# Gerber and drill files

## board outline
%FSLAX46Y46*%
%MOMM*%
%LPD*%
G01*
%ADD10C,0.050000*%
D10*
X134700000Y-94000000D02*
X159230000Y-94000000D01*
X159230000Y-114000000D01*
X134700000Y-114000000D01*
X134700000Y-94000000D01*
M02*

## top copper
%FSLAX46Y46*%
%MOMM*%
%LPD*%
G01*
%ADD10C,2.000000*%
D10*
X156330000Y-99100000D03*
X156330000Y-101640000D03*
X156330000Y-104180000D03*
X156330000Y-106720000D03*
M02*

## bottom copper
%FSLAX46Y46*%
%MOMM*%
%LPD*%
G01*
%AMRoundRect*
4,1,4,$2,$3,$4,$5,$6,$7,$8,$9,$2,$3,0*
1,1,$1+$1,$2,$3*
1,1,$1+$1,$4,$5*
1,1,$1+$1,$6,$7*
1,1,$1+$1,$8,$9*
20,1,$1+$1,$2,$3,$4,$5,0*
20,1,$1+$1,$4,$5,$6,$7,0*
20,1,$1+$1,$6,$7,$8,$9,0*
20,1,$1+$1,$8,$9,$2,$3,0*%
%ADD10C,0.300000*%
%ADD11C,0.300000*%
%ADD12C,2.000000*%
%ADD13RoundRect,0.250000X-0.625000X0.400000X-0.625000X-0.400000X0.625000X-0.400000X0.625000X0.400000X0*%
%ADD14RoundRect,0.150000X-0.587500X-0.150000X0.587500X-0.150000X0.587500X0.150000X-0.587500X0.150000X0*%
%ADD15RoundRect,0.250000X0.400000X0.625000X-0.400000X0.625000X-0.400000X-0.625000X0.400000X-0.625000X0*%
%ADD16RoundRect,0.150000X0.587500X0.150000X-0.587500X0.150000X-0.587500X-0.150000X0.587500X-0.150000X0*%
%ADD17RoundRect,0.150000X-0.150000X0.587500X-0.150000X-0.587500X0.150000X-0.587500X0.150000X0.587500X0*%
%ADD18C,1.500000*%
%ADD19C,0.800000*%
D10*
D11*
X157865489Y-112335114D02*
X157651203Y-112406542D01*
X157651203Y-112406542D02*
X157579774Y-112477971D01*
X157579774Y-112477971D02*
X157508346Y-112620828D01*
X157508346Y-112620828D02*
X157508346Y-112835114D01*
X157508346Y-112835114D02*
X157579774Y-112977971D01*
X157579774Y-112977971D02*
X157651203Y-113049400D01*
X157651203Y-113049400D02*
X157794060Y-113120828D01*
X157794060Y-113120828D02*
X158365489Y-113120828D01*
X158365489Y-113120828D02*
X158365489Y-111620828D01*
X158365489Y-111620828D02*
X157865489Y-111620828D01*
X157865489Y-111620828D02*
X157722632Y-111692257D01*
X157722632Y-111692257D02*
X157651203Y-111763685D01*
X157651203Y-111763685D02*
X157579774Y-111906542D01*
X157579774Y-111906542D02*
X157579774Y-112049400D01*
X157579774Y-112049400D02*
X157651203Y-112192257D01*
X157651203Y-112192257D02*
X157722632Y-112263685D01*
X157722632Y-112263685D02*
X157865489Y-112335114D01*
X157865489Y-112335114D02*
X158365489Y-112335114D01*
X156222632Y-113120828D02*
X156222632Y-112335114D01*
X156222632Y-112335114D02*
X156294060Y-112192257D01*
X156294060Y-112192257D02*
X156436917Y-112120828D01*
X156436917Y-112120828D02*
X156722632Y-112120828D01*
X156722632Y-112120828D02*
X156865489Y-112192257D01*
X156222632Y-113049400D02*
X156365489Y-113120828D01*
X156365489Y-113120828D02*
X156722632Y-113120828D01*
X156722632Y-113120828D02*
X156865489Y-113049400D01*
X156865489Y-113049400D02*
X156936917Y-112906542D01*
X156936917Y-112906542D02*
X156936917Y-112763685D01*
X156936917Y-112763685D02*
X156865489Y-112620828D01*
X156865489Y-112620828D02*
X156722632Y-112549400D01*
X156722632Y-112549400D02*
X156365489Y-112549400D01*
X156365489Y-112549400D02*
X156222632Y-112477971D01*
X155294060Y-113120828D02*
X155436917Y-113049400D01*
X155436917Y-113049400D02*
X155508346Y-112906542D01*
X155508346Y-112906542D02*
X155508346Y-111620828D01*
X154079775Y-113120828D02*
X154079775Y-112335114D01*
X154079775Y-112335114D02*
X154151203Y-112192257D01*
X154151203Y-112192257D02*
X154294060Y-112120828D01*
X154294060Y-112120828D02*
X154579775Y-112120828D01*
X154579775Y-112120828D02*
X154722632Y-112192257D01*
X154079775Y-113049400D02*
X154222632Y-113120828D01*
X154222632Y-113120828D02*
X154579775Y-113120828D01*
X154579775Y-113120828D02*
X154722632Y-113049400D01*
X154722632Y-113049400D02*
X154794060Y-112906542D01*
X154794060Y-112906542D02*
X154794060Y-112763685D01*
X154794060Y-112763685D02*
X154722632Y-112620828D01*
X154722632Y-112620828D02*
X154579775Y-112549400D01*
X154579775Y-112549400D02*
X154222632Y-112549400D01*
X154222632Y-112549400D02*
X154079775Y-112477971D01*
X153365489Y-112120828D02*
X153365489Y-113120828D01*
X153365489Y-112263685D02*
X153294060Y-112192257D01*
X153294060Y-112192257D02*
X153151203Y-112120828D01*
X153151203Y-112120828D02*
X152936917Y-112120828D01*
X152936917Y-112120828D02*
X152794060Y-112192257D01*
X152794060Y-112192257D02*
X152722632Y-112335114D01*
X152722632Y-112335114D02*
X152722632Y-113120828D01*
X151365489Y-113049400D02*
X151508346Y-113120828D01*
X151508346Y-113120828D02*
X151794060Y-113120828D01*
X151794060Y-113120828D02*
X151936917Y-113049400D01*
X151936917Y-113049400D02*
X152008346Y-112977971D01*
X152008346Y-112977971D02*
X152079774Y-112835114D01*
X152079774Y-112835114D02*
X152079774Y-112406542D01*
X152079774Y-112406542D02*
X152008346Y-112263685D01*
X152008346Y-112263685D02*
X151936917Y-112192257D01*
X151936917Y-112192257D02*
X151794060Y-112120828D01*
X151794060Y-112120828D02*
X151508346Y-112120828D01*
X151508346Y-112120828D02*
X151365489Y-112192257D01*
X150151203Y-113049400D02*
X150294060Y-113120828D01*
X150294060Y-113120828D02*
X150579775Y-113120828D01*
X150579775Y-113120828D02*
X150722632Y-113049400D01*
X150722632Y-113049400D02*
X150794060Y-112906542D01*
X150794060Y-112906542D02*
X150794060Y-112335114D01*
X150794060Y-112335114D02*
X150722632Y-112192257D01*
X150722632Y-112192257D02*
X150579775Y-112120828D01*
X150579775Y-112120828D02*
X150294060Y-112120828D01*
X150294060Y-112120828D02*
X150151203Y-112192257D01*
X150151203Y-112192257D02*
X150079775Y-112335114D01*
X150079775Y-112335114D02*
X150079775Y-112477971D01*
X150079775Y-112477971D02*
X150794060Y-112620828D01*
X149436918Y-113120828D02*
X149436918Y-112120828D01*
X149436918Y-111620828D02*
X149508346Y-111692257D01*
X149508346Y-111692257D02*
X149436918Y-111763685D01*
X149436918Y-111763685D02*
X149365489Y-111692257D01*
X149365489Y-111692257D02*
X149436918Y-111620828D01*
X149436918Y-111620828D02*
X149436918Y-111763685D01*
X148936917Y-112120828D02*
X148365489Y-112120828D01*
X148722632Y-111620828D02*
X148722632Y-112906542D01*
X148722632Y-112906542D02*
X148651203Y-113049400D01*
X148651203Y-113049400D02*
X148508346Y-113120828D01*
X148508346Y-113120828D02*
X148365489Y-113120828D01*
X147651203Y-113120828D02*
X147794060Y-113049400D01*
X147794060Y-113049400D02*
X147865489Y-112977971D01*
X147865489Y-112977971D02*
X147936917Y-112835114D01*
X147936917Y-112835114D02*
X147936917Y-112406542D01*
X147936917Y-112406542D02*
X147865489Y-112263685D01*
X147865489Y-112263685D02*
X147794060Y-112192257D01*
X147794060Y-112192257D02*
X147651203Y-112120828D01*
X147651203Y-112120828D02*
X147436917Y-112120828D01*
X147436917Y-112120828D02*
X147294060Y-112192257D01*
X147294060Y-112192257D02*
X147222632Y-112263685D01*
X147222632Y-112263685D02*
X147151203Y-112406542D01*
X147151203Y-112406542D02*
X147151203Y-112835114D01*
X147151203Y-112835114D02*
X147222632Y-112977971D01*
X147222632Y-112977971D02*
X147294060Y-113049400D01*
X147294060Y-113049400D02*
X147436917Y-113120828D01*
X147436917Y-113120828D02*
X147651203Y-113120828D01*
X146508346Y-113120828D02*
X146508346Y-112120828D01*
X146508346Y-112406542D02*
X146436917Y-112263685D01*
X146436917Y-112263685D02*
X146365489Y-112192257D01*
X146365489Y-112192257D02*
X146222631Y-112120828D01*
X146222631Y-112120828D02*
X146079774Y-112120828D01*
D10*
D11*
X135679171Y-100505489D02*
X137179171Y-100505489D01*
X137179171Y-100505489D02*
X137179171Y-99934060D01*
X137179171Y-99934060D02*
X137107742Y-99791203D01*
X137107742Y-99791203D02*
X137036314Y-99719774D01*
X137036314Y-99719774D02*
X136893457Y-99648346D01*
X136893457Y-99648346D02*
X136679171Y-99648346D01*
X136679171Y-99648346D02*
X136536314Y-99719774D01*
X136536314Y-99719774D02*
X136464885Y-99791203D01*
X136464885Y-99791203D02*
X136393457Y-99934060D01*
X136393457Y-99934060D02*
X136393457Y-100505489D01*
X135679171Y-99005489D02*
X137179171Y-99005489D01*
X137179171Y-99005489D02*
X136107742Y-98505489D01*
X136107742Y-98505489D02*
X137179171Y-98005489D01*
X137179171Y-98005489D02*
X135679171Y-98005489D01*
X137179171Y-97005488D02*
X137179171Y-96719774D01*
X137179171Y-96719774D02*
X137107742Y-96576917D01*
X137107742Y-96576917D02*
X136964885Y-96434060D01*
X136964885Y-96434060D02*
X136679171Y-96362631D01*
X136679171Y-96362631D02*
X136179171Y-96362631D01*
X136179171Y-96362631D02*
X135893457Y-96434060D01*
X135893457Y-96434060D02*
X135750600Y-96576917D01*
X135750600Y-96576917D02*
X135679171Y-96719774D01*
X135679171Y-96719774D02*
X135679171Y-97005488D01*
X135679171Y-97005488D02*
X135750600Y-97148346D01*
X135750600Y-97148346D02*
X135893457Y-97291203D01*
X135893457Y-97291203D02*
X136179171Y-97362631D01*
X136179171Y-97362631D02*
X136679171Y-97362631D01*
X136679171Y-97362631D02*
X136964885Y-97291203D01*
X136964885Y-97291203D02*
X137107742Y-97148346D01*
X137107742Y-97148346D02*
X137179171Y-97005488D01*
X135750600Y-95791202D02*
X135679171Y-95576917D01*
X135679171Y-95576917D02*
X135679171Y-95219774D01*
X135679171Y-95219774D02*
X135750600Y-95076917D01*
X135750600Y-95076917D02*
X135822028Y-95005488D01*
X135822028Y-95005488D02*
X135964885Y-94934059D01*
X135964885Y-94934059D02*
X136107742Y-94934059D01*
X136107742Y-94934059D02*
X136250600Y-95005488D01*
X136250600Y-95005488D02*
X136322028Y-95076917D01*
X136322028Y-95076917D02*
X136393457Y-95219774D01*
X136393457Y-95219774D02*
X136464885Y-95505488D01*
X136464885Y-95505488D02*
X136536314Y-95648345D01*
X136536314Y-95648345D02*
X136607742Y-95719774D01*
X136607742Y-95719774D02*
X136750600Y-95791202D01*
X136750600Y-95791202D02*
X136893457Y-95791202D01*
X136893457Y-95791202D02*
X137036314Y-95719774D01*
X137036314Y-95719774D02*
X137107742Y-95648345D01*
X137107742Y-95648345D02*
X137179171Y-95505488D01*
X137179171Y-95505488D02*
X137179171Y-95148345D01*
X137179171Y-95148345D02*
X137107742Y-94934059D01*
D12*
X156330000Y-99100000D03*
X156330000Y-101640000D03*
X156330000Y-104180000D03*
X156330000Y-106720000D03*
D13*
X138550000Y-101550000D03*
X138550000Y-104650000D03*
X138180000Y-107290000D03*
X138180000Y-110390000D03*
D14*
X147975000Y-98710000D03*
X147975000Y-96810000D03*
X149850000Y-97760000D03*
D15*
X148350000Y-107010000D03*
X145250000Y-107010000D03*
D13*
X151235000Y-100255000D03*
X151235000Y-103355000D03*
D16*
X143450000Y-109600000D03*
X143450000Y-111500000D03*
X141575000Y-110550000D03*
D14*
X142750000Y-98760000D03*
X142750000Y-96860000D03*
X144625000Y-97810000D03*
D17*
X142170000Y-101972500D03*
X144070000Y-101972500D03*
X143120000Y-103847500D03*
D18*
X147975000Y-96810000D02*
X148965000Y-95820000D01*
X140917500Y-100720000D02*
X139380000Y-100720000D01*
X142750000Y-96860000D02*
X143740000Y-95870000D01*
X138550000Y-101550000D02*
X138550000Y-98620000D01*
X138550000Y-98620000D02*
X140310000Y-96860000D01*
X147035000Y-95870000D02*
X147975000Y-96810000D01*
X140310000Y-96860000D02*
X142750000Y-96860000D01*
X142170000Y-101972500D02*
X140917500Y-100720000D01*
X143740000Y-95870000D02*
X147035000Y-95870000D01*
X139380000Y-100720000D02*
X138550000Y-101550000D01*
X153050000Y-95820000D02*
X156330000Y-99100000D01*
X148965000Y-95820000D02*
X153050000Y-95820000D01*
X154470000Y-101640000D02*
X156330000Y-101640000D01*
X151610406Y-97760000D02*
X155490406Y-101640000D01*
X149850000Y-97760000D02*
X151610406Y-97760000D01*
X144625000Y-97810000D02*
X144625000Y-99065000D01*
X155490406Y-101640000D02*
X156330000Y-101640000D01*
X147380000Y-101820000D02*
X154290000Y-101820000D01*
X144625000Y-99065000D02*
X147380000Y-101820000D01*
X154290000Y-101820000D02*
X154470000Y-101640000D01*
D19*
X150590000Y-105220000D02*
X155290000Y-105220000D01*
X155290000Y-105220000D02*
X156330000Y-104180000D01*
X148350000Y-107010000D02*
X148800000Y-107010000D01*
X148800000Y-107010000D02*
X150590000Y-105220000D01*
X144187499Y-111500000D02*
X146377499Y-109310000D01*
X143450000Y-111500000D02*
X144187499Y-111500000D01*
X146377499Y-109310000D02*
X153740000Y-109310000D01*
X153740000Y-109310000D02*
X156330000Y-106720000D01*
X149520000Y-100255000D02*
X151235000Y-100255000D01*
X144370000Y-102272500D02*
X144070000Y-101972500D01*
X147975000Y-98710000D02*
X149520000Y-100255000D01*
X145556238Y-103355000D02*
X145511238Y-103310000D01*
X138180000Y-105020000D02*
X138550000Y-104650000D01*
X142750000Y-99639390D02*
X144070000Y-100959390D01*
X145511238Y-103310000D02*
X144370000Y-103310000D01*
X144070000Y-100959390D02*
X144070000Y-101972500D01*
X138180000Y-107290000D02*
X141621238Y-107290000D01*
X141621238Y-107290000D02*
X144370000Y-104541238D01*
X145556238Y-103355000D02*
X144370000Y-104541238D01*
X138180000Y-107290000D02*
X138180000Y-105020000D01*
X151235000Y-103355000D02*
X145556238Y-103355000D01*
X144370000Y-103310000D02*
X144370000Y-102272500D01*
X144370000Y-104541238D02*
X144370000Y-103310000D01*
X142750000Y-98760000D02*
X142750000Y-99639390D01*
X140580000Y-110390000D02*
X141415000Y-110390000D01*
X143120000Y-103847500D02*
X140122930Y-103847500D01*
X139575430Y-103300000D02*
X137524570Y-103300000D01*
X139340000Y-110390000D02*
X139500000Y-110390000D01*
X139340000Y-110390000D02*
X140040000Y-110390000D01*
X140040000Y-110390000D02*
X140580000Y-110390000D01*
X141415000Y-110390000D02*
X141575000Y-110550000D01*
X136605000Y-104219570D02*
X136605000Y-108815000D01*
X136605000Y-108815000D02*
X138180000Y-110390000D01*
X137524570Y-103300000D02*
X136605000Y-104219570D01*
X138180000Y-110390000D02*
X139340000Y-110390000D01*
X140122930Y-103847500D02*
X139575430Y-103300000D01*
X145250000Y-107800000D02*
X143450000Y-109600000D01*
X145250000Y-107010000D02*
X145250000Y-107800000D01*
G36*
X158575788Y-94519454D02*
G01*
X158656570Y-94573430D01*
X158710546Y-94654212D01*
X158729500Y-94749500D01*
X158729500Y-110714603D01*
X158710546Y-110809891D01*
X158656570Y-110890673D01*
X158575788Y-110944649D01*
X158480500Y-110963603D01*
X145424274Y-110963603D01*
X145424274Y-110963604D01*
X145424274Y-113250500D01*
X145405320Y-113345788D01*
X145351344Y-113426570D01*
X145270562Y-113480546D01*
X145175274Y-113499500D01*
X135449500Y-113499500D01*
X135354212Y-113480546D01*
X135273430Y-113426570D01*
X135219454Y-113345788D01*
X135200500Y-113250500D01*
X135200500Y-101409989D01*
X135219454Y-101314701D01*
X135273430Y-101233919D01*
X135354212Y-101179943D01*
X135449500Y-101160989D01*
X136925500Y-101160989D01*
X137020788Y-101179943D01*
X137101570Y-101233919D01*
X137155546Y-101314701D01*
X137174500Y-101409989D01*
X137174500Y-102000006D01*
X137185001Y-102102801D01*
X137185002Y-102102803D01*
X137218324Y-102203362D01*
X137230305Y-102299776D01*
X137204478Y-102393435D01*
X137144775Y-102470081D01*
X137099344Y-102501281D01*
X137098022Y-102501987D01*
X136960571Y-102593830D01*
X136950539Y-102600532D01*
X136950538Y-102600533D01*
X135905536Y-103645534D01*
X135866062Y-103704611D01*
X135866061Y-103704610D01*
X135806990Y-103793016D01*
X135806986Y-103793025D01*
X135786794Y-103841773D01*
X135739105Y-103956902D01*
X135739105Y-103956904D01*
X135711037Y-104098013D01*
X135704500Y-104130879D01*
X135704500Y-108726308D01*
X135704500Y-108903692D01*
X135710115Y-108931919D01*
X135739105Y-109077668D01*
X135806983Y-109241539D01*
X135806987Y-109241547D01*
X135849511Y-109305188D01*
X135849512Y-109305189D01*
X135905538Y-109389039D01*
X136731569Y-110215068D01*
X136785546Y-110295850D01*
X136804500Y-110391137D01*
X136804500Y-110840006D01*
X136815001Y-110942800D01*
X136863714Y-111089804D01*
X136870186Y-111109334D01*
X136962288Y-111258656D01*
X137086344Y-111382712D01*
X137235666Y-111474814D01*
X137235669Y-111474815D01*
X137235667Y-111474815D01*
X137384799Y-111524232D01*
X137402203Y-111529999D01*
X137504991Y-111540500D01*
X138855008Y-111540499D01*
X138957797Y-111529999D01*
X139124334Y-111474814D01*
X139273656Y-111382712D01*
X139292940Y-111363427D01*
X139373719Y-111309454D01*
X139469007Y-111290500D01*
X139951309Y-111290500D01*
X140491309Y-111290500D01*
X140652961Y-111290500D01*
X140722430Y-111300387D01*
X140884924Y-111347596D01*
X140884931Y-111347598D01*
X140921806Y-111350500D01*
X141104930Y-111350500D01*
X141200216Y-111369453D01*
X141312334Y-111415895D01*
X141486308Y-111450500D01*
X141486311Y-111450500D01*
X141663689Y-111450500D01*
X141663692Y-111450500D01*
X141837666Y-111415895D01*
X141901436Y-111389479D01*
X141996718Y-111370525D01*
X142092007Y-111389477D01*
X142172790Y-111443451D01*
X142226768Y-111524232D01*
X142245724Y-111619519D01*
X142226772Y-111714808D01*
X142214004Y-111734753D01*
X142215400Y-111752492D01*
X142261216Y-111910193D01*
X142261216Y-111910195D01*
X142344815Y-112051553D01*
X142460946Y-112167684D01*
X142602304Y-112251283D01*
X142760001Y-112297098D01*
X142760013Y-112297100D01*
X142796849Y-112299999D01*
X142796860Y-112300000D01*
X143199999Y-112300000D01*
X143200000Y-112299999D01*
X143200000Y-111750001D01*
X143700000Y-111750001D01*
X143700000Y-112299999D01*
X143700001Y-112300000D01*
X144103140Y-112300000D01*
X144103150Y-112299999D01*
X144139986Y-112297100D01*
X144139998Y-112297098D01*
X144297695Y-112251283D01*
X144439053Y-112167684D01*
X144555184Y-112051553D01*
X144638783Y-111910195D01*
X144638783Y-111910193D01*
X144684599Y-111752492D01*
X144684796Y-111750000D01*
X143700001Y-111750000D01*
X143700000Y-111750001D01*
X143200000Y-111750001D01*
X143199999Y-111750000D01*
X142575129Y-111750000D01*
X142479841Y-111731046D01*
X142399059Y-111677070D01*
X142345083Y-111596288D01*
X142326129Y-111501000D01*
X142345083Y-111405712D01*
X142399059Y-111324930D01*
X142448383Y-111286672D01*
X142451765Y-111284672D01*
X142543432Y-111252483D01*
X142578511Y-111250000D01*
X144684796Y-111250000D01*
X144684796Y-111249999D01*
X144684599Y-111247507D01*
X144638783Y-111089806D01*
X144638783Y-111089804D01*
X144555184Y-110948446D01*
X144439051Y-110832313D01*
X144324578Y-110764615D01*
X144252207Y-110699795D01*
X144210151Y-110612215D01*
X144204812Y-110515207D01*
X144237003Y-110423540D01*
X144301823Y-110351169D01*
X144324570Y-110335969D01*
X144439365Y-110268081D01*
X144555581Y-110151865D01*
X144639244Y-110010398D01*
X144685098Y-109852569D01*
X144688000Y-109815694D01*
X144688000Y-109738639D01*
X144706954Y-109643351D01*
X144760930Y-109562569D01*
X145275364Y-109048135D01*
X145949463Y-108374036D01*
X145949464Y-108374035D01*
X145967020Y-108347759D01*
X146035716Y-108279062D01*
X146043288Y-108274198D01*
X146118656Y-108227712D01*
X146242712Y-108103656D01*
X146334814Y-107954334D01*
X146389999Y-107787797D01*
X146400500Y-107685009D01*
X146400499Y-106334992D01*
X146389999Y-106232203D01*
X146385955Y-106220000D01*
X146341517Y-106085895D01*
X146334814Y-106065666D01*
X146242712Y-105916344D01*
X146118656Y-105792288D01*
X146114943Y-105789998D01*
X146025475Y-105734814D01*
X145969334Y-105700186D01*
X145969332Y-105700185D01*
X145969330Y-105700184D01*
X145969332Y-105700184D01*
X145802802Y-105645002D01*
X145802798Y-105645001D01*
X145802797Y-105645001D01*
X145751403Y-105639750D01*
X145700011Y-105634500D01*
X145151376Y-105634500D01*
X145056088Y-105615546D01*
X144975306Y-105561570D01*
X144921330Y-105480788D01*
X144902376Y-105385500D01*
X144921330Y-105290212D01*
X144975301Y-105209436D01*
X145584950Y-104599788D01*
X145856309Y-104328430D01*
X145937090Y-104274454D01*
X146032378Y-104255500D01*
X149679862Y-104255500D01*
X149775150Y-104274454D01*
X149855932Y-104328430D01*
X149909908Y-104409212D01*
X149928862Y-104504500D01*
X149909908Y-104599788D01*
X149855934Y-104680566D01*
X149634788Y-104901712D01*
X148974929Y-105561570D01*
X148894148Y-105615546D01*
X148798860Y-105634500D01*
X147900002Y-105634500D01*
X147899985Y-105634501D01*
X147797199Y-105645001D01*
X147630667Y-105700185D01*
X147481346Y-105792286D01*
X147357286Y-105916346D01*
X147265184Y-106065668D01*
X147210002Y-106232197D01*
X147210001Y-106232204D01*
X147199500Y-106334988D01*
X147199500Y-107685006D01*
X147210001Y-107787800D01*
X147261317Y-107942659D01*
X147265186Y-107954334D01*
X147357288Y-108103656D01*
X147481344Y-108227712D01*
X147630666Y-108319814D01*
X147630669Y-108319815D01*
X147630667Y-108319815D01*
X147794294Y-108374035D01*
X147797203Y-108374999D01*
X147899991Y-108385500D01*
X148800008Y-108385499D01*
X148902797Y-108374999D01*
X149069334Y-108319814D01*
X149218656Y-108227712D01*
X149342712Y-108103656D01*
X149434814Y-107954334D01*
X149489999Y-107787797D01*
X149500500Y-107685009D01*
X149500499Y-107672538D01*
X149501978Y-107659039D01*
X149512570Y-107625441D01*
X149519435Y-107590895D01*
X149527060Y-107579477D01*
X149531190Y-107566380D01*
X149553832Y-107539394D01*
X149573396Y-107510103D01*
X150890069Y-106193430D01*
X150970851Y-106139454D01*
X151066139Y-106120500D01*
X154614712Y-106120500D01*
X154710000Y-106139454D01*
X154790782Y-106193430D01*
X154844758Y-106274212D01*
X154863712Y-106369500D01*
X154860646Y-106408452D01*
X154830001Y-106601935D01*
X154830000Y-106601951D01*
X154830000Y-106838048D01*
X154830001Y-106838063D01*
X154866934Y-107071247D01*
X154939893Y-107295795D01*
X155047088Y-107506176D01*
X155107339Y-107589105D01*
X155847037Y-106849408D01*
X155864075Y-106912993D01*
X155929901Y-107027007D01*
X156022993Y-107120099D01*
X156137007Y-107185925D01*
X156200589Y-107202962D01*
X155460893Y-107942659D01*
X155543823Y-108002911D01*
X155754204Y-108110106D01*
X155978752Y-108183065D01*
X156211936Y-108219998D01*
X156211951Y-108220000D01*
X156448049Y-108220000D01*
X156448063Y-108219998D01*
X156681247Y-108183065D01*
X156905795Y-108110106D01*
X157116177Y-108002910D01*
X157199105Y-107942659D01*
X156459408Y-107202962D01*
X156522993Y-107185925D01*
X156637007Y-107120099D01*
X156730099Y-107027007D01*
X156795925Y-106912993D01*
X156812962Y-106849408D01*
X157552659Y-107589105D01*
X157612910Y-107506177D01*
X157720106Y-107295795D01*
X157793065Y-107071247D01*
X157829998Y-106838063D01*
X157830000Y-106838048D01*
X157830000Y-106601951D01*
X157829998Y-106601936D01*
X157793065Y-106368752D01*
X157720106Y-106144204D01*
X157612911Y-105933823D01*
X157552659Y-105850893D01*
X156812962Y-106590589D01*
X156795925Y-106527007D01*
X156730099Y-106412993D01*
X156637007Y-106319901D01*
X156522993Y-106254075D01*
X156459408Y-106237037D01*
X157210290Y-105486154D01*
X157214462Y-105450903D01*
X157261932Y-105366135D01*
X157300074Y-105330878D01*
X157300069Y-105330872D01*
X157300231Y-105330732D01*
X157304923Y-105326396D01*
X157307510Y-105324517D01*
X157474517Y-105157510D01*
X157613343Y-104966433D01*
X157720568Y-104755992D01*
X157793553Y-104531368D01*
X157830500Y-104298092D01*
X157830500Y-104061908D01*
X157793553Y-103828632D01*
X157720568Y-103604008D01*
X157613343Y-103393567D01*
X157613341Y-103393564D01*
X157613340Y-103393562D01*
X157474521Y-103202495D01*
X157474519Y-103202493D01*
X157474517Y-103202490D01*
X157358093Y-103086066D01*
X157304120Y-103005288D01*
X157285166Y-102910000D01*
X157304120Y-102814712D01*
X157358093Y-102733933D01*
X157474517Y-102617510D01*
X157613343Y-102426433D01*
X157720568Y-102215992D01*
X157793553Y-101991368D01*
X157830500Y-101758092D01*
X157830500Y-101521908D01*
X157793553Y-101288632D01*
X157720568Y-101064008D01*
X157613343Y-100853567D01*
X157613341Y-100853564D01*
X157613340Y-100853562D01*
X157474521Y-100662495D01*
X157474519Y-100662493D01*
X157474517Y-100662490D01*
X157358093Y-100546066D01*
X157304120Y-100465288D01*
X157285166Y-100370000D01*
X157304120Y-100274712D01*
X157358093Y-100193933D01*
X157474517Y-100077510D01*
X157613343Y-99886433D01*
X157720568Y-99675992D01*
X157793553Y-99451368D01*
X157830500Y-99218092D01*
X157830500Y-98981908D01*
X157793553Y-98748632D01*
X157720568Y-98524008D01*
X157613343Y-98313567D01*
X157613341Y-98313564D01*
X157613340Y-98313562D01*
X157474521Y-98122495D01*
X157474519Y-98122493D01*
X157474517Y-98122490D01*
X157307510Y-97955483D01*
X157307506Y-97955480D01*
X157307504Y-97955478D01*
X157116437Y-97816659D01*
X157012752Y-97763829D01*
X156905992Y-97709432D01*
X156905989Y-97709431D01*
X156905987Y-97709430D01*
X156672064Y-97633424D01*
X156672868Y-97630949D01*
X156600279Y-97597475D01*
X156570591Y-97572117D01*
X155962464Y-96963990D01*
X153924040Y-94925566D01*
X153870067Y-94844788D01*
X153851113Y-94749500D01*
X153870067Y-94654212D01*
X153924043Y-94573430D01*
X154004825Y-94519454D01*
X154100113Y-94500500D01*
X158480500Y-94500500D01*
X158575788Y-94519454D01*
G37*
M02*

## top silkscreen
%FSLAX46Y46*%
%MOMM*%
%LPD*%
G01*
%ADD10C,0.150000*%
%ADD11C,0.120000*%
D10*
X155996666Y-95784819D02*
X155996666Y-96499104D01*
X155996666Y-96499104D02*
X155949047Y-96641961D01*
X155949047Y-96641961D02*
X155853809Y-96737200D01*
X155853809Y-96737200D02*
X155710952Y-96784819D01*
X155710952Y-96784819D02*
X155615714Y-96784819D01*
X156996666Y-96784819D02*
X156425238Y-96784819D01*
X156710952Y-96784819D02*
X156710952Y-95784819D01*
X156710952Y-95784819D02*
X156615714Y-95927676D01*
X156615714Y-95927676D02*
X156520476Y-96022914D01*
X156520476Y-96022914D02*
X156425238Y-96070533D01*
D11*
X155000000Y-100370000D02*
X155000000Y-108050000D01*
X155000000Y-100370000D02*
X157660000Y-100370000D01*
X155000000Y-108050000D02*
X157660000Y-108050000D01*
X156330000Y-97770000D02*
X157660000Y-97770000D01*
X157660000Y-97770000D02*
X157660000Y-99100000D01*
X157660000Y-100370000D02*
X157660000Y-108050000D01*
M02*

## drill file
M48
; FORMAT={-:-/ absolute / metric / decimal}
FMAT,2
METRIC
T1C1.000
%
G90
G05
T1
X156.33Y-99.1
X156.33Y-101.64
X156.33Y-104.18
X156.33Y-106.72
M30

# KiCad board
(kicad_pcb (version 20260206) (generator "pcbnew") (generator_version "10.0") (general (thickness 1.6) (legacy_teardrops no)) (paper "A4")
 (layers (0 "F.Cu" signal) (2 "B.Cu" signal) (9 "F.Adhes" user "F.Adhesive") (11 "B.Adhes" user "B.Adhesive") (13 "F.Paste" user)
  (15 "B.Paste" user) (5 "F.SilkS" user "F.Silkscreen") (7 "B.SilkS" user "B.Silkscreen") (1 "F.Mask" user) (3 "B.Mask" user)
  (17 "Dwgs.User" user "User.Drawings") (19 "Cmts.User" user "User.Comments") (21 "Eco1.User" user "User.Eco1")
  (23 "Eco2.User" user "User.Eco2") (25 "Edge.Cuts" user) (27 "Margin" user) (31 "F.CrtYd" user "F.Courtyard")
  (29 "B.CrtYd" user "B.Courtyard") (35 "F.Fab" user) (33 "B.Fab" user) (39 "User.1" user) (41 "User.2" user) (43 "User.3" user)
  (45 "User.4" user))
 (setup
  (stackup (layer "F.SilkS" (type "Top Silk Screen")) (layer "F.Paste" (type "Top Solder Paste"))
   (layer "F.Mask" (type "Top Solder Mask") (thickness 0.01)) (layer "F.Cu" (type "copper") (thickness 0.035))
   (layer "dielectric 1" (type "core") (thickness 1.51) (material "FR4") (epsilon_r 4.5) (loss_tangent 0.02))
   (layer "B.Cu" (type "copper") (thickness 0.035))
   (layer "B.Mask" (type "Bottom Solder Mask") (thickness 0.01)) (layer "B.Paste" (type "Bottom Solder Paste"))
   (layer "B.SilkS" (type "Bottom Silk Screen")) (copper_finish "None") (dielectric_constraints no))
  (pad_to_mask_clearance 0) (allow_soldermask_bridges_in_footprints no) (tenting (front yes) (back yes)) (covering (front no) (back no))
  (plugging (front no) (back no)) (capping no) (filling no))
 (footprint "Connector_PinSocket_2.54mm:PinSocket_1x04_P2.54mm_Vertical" (layer "F.Cu") (at 156.33 99.1)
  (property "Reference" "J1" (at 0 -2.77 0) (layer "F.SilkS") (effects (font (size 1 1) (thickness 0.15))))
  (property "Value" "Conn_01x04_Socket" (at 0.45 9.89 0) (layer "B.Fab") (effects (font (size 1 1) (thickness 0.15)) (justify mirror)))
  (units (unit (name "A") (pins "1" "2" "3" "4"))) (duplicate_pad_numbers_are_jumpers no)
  (fp_line (start -1.33 1.27) (end -1.33 8.95) (stroke (width 0.12) (type solid)) (layer "F.SilkS"))
  (fp_line (start -1.33 1.27) (end 1.33 1.27) (stroke (width 0.12) (type solid)) (layer "F.SilkS"))
  (fp_line (start -1.33 8.95) (end 1.33 8.95) (stroke (width 0.12) (type solid)) (layer "F.SilkS"))
  (fp_line (start 0 -1.33) (end 1.33 -1.33) (stroke (width 0.12) (type solid)) (layer "F.SilkS"))
  (fp_line (start 1.33 -1.33) (end 1.33 0) (stroke (width 0.12) (type solid)) (layer "F.SilkS"))
  (fp_line (start 1.33 1.27) (end 1.33 8.95) (stroke (width 0.12) (type solid)) (layer "F.SilkS"))
  (pad "1" thru_hole circle (at 0 0) (size 2 2) (drill 1) (layers "*.Cu" "*.Mask") (remove_unused_layers no) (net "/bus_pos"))
  (pad "2" thru_hole circle (at 0 2.54) (size 2 2) (drill 1) (layers "*.Cu" "*.Mask") (remove_unused_layers no) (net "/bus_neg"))
  (pad "3" thru_hole circle (at 0 5.08) (size 2 2) (drill 1) (layers "*.Cu" "*.Mask") (remove_unused_layers no) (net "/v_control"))
  (pad "4" thru_hole circle (at 0 7.62) (size 2 2) (drill 1) (layers "*.Cu" "*.Mask") (remove_unused_layers no) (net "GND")))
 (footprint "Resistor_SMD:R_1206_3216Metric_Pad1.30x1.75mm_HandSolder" (layer "B.Cu") (at 138.55 103.1 -90)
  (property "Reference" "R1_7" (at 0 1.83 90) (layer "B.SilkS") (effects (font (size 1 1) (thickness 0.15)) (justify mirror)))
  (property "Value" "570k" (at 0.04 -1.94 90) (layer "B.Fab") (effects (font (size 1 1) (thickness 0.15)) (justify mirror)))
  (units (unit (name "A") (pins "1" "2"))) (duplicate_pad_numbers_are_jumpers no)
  (pad "1" smd roundrect (at -1.55 0 270) (size 1.3 1.75) (layers "B.Cu" "B.Mask" "B.Paste") (roundrect_rratio 0.192308) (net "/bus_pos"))
  (pad "2" smd roundrect (at 1.55 0 270) (size 1.3 1.75) (layers "B.Cu" "B.Mask" "B.Paste") (roundrect_rratio 0.192308) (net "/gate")))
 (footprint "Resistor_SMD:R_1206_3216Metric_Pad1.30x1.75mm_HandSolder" (layer "B.Cu") (at 138.18 108.84 -90)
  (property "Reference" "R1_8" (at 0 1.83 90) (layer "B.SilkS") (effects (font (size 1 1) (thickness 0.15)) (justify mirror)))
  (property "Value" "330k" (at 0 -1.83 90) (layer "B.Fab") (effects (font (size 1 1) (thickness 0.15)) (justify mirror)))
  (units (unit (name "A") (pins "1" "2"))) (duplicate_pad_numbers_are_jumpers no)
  (pad "1" smd roundrect (at -1.55 0 270) (size 1.3 1.75) (layers "B.Cu" "B.Mask" "B.Paste") (roundrect_rratio 0.192308) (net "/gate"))
  (pad "2" smd roundrect (at 1.55 0 270) (size 1.3 1.75) (layers "B.Cu" "B.Mask" "B.Paste") (roundrect_rratio 0.192308) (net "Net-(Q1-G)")))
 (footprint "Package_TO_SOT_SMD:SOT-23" (layer "B.Cu") (at 148.9125 97.76)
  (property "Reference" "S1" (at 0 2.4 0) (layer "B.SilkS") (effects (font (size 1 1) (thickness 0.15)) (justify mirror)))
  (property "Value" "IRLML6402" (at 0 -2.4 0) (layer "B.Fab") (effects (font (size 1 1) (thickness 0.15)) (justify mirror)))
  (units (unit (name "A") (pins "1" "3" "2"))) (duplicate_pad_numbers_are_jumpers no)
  (pad "1" smd roundrect (at -0.9375 0.95) (size 1.475 0.6) (layers "B.Cu" "B.Mask" "B.Paste") (roundrect_rratio 0.25) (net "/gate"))
  (pad "2" smd roundrect (at -0.9375 -0.95) (size 1.475 0.6) (layers "B.Cu" "B.Mask" "B.Paste") (roundrect_rratio 0.25) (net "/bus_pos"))
  (pad "3" smd roundrect (at 0.9375 0) (size 1.475 0.6) (layers "B.Cu" "B.Mask" "B.Paste") (roundrect_rratio 0.25) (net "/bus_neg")))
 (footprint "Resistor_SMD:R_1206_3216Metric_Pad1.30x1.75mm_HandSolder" (layer "B.Cu") (at 146.8 107.01 180)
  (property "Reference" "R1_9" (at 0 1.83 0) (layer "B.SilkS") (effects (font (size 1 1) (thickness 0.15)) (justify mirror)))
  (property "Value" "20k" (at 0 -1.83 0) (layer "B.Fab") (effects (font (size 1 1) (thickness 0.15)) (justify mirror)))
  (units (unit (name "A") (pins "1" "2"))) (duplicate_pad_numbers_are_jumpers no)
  (pad "1" smd roundrect (at -1.55 0 180) (size 1.3 1.75) (layers "B.Cu" "B.Mask" "B.Paste") (roundrect_rratio 0.192308) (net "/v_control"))
  (pad "2" smd roundrect (at 1.55 0 180) (size 1.3 1.75) (layers "B.Cu" "B.Mask" "B.Paste") (roundrect_rratio 0.192308) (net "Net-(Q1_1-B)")))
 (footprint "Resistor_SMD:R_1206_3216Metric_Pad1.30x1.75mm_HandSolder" (layer "B.Cu") (at 151.235 101.805 -90)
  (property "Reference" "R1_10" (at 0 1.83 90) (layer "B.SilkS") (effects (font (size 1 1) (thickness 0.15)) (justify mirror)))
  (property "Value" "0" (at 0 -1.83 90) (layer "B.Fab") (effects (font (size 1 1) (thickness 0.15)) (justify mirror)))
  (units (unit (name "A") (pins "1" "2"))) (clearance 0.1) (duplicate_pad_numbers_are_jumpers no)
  (pad "1" smd roundrect (at -1.55 0 270) (size 1.3 1.75) (layers "B.Cu" "B.Mask" "B.Paste") (roundrect_rratio 0.192308) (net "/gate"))
  (pad "2" smd roundrect (at 1.55 0 270) (size 1.3 1.75) (layers "B.Cu" "B.Mask" "B.Paste") (roundrect_rratio 0.192308) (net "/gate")))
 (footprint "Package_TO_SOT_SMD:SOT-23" (layer "B.Cu") (at 142.5125 110.55 180)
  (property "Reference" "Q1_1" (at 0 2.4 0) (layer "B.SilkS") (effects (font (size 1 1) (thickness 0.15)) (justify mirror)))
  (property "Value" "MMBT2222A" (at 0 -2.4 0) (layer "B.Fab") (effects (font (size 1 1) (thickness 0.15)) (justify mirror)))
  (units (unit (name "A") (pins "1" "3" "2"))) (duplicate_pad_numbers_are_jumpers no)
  (pad "1" smd roundrect (at -0.9375 0.95 180) (size 1.475 0.6) (layers "B.Cu" "B.Mask" "B.Paste") (roundrect_rratio 0.25)
   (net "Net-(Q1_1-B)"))
  (pad "2" smd roundrect (at -0.9375 -0.95 180) (size 1.475 0.6) (layers "B.Cu" "B.Mask" "B.Paste") (roundrect_rratio 0.25) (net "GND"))
  (pad "3" smd roundrect (at 0.9375 0 180) (size 1.475 0.6) (layers "B.Cu" "B.Mask" "B.Paste") (roundrect_rratio 0.25) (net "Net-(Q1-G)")))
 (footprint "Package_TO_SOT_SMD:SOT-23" (layer "B.Cu") (at 143.6875 97.81)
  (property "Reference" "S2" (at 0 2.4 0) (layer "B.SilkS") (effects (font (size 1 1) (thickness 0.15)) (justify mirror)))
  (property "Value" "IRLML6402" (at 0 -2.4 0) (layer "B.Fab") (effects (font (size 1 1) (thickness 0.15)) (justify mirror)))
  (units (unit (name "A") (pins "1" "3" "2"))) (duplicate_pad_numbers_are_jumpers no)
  (pad "1" smd roundrect (at -0.9375 0.95) (size 1.475 0.6) (layers "B.Cu" "B.Mask" "B.Paste") (roundrect_rratio 0.25) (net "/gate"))
  (pad "2" smd roundrect (at -0.9375 -0.95) (size 1.475 0.6) (layers "B.Cu" "B.Mask" "B.Paste") (roundrect_rratio 0.25) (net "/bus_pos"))
  (pad "3" smd roundrect (at 0.9375 0) (size 1.475 0.6) (layers "B.Cu" "B.Mask" "B.Paste") (roundrect_rratio 0.25) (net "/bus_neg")))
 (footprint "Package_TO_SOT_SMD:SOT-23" (layer "B.Cu") (at 143.12 102.91 -90)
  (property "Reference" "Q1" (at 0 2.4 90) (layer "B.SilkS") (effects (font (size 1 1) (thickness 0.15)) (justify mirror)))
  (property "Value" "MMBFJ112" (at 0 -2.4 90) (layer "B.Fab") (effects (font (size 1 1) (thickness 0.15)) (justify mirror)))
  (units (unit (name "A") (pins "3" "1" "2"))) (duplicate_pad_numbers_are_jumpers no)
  (pad "1" smd roundrect (at -0.9375 0.95 270) (size 1.475 0.6) (layers "B.Cu" "B.Mask" "B.Paste") (roundrect_rratio 0.25) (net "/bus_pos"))
  (pad "2" smd roundrect (at -0.9375 -0.95 270) (size 1.475 0.6) (layers "B.Cu" "B.Mask" "B.Paste") (roundrect_rratio 0.25) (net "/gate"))
  (pad "3" smd roundrect (at 0.9375 0 270) (size 1.475 0.6) (layers "B.Cu" "B.Mask" "B.Paste") (roundrect_rratio 0.25) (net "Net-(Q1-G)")))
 (gr_rect (start 134.7 94) (end 159.23 114) (stroke (width 0.05) (type solid)) (fill no) (layer "Edge.Cuts"))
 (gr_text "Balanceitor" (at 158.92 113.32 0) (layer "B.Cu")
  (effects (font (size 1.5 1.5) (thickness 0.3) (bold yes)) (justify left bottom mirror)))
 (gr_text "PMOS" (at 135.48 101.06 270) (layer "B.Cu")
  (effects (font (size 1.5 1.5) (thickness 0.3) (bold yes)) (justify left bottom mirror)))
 (segment (start 147.975 96.81) (end 148.965 95.82) (width 1.5) (layer "B.Cu") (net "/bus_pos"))
 (segment (start 140.9175 100.72) (end 139.38 100.72) (width 1.5) (layer "B.Cu") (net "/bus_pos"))
 (segment (start 142.75 96.86) (end 143.74 95.87) (width 1.5) (layer "B.Cu") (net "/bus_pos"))
 (segment (start 138.55 101.55) (end 138.55 98.62) (width 1.5) (layer "B.Cu") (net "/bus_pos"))
 (segment (start 138.55 98.62) (end 140.31 96.86) (width 1.5) (layer "B.Cu") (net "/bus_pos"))
 (segment (start 147.035 95.87) (end 147.975 96.81) (width 1.5) (layer "B.Cu") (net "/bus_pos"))
 (segment (start 140.31 96.86) (end 142.75 96.86) (width 1.5) (layer "B.Cu") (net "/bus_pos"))
 (segment (start 142.17 101.9725) (end 140.9175 100.72) (width 1.5) (layer "B.Cu") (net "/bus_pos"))
 (segment (start 143.74 95.87) (end 147.035 95.87) (width 1.5) (layer "B.Cu") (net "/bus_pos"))
 (segment (start 139.38 100.72) (end 138.55 101.55) (width 1.5) (layer "B.Cu") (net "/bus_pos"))
 (segment (start 153.05 95.82) (end 156.33 99.1) (width 1.5) (layer "B.Cu") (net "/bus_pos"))
 (segment (start 148.965 95.82) (end 153.05 95.82) (width 1.5) (layer "B.Cu") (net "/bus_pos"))
 (segment (start 154.47 101.64) (end 156.33 101.64) (width 1.5) (layer "B.Cu") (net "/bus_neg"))
 (segment (start 151.610406 97.76) (end 155.490406 101.64) (width 1.5) (layer "B.Cu") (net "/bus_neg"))
 (segment (start 149.85 97.76) (end 151.610406 97.76) (width 1.5) (layer "B.Cu") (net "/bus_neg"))
 (segment (start 144.625 97.81) (end 144.625 99.065) (width 1.5) (layer "B.Cu") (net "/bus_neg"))
 (segment (start 155.490406 101.64) (end 156.33 101.64) (width 1.5) (layer "B.Cu") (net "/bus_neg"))
 (segment (start 147.38 101.82) (end 154.29 101.82) (width 1.5) (layer "B.Cu") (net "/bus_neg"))
 (segment (start 144.625 99.065) (end 147.38 101.82) (width 1.5) (layer "B.Cu") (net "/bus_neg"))
 (segment (start 154.29 101.82) (end 154.47 101.64) (width 1.5) (layer "B.Cu") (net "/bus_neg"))
 (segment (start 150.59 105.22) (end 155.29 105.22) (width 0.8) (layer "B.Cu") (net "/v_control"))
 (segment (start 155.29 105.22) (end 156.33 104.18) (width 0.8) (layer "B.Cu") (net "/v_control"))
 (segment (start 148.35 107.01) (end 148.8 107.01) (width 0.8) (layer "B.Cu") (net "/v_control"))
 (segment (start 148.8 107.01) (end 150.59 105.22) (width 0.8) (layer "B.Cu") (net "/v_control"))
 (segment (start 144.187499 111.5) (end 146.377499 109.31) (width 0.8) (layer "B.Cu") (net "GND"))
 (segment (start 143.45 111.5) (end 144.187499 111.5) (width 0.8) (layer "B.Cu") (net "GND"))
 (segment (start 146.377499 109.31) (end 153.74 109.31) (width 0.8) (layer "B.Cu") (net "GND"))
 (segment (start 153.74 109.31) (end 156.33 106.72) (width 0.8) (layer "B.Cu") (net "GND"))
 (segment (start 149.52 100.255) (end 151.235 100.255) (width 0.8) (layer "B.Cu") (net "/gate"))
 (segment (start 144.37 102.2725) (end 144.07 101.9725) (width 0.8) (layer "B.Cu") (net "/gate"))
 (segment (start 147.975 98.71) (end 149.52 100.255) (width 0.8) (layer "B.Cu") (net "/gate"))
 (segment (start 145.556238 103.355) (end 145.511238 103.31) (width 0.8) (layer "B.Cu") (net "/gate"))
 (segment (start 138.18 105.02) (end 138.55 104.65) (width 0.8) (layer "B.Cu") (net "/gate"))
 (segment (start 142.75 99.63939) (end 144.07 100.95939) (width 0.8) (layer "B.Cu") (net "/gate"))
 (segment (start 145.511238 103.31) (end 144.37 103.31) (width 0.8) (layer "B.Cu") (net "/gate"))
 (segment (start 144.07 100.95939) (end 144.07 101.9725) (width 0.8) (layer "B.Cu") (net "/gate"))
 (segment (start 138.18 107.29) (end 141.621238 107.29) (width 0.8) (layer "B.Cu") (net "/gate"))
 (segment (start 141.621238 107.29) (end 144.37 104.541238) (width 0.8) (layer "B.Cu") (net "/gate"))
 (segment (start 145.556238 103.355) (end 144.37 104.541238) (width 0.8) (layer "B.Cu") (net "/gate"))
 (segment (start 138.18 107.29) (end 138.18 105.02) (width 0.8) (layer "B.Cu") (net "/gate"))
 (segment (start 151.235 103.355) (end 145.556238 103.355) (width 0.8) (layer "B.Cu") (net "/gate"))
 (segment (start 144.37 103.31) (end 144.37 102.2725) (width 0.8) (layer "B.Cu") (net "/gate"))
 (segment (start 144.37 104.541238) (end 144.37 103.31) (width 0.8) (layer "B.Cu") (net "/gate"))
 (segment (start 142.75 98.76) (end 142.75 99.63939) (width 0.8) (layer "B.Cu") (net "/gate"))
 (segment (start 140.58 110.39) (end 141.415 110.39) (width 0.8) (layer "B.Cu") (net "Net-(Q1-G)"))
 (segment (start 143.12 103.8475) (end 140.12293 103.8475) (width 0.8) (layer "B.Cu") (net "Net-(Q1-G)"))
 (segment (start 139.57543 103.3) (end 137.52457 103.3) (width 0.8) (layer "B.Cu") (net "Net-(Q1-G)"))
 (segment (start 139.34 110.39) (end 139.5 110.39) (width 0.8) (layer "B.Cu") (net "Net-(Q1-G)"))
 (segment (start 139.34 110.39) (end 140.04 110.39) (width 0.8) (layer "B.Cu") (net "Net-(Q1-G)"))
 (segment (start 140.04 110.39) (end 140.58 110.39) (width 0.8) (layer "B.Cu") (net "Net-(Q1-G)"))
 (segment (start 141.415 110.39) (end 141.575 110.55) (width 0.8) (layer "B.Cu") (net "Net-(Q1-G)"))
 (segment (start 136.605 104.21957) (end 136.605 108.815) (width 0.8) (layer "B.Cu") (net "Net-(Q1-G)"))
 (segment (start 136.605 108.815) (end 138.18 110.39) (width 0.8) (layer "B.Cu") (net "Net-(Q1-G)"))
 (segment (start 137.52457 103.3) (end 136.605 104.21957) (width 0.8) (layer "B.Cu") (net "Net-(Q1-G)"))
 (segment (start 138.18 110.39) (end 139.34 110.39) (width 0.8) (layer "B.Cu") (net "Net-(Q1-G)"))
 (segment (start 140.12293 103.8475) (end 139.57543 103.3) (width 0.8) (layer "B.Cu") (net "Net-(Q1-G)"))
 (segment (start 145.25 107.8) (end 143.45 109.6) (width 0.8) (layer "B.Cu") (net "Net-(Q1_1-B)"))
 (segment (start 145.25 107.01) (end 145.25 107.8) (width 0.8) (layer "B.Cu") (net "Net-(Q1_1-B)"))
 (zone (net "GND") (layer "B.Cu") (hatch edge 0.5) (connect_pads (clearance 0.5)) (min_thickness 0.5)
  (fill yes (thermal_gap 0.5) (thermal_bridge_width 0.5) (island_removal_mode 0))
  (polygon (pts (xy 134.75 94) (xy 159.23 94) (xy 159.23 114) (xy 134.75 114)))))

